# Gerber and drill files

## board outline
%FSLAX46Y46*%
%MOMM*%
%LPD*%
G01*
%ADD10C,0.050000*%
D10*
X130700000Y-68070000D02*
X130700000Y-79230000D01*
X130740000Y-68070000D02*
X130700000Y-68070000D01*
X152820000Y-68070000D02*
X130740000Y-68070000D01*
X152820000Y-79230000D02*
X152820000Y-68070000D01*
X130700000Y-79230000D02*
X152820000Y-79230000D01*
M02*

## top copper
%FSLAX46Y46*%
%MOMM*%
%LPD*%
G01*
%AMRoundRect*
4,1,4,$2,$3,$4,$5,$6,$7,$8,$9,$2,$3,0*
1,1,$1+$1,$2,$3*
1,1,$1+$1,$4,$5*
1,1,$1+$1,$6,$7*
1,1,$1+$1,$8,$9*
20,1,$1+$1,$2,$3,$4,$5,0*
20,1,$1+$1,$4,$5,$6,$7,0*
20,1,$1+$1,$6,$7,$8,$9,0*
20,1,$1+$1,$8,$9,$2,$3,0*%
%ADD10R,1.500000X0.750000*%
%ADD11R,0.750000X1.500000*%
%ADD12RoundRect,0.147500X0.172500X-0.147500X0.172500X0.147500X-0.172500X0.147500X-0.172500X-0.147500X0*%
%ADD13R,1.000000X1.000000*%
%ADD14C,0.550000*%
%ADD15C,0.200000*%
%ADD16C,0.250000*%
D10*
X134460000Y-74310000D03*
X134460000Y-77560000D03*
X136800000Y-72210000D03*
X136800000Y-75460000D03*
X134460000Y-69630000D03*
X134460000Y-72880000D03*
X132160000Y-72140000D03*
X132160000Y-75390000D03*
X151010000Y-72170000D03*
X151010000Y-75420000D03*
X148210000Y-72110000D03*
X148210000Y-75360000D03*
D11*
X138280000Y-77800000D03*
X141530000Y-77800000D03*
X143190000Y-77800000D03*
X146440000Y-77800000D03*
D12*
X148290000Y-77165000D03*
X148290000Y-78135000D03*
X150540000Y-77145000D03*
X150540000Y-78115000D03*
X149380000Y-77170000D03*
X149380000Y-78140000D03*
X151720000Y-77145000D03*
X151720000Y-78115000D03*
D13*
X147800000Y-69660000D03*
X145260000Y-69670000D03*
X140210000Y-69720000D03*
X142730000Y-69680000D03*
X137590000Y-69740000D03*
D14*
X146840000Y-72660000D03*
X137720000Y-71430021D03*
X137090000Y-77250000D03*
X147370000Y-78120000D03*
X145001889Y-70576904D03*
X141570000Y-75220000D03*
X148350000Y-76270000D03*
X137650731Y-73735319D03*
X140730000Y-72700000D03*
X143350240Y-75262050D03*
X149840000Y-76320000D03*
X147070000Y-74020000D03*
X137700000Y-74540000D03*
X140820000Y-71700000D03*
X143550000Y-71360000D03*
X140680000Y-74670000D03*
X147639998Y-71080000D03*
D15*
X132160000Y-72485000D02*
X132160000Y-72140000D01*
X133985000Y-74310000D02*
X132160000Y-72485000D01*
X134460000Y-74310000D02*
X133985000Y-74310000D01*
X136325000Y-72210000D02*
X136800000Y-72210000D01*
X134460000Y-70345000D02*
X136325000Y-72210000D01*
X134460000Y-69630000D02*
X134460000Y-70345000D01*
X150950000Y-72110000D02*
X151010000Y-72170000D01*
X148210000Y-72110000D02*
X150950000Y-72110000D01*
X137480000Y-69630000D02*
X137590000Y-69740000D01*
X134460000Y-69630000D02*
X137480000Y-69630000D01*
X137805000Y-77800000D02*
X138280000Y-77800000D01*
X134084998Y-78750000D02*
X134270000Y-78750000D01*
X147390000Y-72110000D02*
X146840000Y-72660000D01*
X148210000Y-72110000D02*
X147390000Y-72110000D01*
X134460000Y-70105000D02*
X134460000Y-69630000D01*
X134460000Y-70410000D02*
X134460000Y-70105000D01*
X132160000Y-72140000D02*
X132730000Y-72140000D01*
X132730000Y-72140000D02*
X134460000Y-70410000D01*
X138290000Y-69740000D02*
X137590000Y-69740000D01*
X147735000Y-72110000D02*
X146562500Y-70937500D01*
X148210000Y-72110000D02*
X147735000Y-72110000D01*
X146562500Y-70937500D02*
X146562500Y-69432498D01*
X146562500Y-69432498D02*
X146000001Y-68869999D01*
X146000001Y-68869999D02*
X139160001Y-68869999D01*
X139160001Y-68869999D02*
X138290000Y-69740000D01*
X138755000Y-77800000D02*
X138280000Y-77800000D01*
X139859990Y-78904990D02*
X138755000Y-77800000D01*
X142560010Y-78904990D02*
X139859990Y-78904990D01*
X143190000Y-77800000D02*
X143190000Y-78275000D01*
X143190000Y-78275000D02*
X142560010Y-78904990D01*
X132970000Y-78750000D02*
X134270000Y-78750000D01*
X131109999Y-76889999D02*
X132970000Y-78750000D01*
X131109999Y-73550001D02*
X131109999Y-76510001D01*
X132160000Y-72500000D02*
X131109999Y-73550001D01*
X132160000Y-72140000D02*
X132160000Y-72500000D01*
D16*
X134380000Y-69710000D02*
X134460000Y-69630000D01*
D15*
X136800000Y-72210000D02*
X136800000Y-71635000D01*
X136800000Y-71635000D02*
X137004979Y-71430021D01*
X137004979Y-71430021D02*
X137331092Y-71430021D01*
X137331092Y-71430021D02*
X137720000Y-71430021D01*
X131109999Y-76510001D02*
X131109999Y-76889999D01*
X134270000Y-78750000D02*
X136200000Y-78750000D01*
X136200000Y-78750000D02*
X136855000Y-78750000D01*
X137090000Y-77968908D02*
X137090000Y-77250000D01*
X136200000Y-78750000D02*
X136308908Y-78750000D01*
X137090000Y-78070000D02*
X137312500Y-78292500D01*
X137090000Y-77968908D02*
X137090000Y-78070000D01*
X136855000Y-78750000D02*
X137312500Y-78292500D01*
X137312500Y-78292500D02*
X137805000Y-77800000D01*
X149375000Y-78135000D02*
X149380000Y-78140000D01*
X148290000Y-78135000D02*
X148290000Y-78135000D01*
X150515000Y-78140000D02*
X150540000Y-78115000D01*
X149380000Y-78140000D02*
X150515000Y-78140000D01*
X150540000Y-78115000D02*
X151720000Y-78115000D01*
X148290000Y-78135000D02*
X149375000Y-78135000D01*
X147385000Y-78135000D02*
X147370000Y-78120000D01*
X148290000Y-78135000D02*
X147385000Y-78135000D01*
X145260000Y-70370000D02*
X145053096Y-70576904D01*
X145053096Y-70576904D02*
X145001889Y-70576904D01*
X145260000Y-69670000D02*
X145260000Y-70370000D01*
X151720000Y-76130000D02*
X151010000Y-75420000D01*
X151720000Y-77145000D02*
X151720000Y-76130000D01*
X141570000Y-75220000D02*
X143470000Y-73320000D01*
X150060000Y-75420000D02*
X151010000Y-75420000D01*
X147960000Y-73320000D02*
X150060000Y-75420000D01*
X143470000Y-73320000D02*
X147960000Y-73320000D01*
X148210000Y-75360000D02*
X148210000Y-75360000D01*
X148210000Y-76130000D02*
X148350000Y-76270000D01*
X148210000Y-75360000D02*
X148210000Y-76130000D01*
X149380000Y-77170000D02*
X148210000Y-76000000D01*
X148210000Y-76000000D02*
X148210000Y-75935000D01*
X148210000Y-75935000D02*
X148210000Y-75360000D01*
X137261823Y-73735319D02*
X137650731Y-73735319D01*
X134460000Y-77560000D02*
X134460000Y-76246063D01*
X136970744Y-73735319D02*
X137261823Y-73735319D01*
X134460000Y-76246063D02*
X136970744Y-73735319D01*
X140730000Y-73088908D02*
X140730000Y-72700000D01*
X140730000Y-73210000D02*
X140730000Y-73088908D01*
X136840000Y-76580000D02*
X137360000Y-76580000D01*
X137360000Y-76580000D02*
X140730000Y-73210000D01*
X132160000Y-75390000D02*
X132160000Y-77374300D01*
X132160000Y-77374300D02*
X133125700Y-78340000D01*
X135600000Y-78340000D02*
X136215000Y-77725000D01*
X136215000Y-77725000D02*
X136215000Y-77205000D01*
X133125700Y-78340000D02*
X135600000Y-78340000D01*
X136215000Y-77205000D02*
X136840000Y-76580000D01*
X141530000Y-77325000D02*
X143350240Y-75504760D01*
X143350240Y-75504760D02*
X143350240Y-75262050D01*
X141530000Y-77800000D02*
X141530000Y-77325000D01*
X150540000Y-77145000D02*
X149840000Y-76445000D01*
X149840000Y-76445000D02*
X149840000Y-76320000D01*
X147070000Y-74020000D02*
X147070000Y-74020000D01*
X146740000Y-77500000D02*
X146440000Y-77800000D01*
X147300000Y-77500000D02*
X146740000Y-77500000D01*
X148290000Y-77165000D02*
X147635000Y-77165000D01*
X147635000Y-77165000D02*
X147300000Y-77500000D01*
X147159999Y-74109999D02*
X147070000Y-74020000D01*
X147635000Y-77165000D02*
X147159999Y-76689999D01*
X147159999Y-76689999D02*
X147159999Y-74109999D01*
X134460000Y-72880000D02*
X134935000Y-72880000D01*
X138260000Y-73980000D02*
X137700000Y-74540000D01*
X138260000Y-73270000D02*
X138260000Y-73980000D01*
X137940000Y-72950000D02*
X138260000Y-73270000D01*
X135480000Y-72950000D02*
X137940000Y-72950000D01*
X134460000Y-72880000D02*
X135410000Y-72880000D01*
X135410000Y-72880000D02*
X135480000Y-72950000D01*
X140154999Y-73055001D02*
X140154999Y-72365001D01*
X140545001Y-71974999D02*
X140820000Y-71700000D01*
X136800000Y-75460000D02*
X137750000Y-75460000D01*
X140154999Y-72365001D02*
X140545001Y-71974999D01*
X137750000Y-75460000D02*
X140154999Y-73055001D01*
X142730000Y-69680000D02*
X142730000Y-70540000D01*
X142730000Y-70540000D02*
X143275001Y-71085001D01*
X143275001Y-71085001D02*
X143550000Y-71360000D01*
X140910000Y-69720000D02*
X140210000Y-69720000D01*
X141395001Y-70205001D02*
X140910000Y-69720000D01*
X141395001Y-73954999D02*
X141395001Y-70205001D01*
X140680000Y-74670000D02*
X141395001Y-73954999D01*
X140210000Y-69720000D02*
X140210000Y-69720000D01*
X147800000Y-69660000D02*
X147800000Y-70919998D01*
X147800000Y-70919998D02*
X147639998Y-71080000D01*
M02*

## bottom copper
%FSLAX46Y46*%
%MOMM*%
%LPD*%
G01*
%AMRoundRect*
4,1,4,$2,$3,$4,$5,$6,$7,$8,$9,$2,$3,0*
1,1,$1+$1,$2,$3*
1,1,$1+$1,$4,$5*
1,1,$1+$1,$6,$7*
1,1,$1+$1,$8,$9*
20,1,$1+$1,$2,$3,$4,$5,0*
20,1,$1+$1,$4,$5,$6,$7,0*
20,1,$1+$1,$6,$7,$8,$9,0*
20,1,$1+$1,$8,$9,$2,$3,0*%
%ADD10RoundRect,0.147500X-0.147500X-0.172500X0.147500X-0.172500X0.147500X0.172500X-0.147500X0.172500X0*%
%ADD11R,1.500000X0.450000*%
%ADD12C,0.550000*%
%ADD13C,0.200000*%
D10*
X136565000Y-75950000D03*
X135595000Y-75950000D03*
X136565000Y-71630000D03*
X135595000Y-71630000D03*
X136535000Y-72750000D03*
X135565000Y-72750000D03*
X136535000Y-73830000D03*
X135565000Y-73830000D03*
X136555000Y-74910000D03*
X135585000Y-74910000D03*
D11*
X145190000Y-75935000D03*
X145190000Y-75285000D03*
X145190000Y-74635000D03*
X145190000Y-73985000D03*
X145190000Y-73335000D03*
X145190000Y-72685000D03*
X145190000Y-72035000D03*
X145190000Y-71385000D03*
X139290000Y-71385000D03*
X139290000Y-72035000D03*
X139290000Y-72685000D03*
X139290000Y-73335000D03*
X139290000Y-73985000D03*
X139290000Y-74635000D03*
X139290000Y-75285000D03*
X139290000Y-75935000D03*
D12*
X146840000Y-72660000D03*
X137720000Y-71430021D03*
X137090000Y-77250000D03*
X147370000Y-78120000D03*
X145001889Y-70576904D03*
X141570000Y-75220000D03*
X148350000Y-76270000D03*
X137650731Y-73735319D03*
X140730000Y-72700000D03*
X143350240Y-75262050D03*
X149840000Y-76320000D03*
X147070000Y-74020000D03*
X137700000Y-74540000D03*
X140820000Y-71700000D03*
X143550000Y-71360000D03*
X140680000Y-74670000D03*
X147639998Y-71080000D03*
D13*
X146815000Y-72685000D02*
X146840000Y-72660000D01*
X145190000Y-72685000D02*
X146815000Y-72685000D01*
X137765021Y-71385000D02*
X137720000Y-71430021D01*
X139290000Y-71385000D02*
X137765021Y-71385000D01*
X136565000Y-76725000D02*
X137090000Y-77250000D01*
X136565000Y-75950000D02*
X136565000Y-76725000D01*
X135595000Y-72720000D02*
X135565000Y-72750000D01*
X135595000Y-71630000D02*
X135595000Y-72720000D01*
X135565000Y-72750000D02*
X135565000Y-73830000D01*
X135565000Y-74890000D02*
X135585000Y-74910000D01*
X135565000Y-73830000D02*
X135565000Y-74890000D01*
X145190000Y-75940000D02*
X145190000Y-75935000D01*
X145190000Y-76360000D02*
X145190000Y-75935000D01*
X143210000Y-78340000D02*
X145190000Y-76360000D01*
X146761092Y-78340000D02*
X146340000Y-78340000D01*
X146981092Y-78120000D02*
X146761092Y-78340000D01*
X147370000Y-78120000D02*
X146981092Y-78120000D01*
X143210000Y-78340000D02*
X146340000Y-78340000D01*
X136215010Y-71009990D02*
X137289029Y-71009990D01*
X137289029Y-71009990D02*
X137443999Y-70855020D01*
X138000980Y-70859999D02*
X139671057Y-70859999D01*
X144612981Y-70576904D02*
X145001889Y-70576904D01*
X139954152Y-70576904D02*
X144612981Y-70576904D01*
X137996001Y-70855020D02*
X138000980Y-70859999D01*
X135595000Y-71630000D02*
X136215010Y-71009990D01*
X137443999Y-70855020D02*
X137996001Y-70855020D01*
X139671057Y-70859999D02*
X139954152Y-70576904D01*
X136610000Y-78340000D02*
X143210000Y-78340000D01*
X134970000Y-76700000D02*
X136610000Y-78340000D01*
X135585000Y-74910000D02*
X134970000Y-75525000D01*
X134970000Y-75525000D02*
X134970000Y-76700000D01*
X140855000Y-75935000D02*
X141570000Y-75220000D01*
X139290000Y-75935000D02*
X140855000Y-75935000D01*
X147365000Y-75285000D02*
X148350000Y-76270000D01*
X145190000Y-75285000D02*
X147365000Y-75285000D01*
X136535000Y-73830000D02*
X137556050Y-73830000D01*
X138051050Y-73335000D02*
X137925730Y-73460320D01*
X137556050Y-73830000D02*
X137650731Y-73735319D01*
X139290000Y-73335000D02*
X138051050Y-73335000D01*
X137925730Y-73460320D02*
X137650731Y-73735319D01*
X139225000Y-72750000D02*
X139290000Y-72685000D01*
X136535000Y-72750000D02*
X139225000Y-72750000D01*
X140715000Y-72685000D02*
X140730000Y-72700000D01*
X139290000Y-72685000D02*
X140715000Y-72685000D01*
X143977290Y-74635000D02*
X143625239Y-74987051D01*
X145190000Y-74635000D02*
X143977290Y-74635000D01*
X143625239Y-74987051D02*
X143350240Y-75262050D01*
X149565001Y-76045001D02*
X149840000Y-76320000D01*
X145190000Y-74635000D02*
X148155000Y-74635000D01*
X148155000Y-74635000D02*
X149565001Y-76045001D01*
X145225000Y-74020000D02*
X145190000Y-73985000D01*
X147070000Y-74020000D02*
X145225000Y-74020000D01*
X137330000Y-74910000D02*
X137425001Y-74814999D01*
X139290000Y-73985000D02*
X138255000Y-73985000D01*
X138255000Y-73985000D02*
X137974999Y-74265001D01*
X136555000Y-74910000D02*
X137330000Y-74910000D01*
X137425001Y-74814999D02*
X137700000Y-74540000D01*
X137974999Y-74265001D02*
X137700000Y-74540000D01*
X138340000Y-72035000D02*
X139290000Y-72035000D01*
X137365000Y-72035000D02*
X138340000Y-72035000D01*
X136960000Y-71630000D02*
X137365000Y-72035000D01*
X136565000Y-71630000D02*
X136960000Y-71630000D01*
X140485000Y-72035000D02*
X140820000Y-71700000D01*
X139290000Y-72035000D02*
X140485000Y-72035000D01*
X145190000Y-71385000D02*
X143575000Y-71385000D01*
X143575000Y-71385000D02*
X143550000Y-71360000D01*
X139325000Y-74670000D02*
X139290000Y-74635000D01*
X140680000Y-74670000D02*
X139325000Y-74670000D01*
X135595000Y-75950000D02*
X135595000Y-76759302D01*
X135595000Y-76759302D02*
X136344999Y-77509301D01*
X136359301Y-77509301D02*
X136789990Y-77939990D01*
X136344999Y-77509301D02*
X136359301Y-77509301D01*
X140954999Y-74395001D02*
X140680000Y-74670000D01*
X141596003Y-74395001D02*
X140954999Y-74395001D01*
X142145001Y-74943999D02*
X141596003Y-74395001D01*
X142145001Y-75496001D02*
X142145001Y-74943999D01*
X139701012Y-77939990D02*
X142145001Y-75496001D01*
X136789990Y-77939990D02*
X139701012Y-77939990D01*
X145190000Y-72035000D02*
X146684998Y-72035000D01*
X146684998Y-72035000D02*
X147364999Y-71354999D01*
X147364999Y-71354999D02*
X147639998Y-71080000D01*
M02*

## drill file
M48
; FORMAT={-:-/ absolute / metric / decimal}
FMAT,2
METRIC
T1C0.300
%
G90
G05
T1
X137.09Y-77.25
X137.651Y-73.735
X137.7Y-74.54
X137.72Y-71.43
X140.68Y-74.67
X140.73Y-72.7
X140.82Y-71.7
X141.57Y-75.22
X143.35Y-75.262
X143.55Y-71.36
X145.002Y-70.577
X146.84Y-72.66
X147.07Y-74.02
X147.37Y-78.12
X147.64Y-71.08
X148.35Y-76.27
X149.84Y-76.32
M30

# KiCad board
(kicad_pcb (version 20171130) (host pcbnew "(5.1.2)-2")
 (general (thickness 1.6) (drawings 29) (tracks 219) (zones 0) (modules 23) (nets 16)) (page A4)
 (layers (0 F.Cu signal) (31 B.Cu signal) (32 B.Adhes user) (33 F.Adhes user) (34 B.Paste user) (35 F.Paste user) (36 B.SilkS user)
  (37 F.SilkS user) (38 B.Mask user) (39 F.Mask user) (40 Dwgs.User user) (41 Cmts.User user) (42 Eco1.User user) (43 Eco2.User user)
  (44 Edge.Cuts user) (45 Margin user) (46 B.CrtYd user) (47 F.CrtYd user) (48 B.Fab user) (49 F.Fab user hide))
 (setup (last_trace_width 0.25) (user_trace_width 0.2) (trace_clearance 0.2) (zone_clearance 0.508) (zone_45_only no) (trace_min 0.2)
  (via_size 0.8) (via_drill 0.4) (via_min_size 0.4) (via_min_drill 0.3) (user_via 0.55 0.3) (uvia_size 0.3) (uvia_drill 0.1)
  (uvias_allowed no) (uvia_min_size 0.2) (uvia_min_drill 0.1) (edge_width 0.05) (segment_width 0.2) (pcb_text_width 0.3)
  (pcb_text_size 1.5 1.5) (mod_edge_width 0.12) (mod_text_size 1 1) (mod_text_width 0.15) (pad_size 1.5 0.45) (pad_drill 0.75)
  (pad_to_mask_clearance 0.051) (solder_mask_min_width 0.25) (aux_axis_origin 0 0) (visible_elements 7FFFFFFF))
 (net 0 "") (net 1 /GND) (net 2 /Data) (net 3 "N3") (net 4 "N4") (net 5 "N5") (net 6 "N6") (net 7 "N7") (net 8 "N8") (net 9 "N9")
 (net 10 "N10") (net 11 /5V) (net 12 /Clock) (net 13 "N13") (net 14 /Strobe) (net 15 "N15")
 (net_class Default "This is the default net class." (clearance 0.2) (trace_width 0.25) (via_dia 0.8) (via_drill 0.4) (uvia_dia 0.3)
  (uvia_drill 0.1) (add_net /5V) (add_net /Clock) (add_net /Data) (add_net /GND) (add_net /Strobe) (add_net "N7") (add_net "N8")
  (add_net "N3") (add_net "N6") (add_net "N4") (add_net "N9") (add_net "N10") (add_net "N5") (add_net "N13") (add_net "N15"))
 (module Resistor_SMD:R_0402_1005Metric (layer B.Cu) (at 136.08 75.95)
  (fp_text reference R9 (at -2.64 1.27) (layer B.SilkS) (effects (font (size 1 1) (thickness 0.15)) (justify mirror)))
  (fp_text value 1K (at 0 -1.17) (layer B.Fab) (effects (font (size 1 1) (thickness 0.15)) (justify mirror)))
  (pad 2 smd roundrect (at 0.485 0) (size 0.59 0.64) (layers B.Cu B.Paste B.Mask) (roundrect_rratio 0.25) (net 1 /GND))
  (pad 1 smd roundrect (at -0.485 0) (size 0.59 0.64) (layers B.Cu B.Paste B.Mask) (roundrect_rratio 0.25) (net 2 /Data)))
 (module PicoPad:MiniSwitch (layer F.Cu) (at 131.92 78.83 90)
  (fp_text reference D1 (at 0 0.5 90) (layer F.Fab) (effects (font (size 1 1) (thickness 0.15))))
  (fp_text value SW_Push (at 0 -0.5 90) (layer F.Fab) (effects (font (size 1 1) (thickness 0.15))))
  (pad 1 smd rect (at 4.52 2.54 90) (size 0.75 1.5) (layers F.Cu F.Paste F.Mask) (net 1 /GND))
  (pad 2 smd rect (at 1.27 2.54 90) (size 0.75 1.5) (layers F.Cu F.Paste F.Mask) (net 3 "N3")))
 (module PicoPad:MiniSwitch (layer F.Cu) (at 134.26 76.73 90)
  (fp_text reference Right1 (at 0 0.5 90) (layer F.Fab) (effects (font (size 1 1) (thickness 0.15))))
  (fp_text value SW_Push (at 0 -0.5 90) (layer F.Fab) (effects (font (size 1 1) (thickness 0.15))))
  (pad 1 smd rect (at 4.52 2.54 90) (size 0.75 1.5) (layers F.Cu F.Paste F.Mask) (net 1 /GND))
  (pad 2 smd rect (at 1.27 2.54 90) (size 0.75 1.5) (layers F.Cu F.Paste F.Mask) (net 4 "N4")))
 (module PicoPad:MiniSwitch (layer F.Cu) (at 131.92 74.15 90)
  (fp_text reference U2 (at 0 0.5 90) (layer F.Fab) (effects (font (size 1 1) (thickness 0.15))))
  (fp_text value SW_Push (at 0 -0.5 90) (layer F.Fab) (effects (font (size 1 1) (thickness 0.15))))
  (pad 1 smd rect (at 4.52 2.54 90) (size 0.75 1.5) (layers F.Cu F.Paste F.Mask) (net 1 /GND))
  (pad 2 smd rect (at 1.27 2.54 90) (size 0.75 1.5) (layers F.Cu F.Paste F.Mask) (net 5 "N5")))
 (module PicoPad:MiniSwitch (layer F.Cu) (at 129.62 76.66 90)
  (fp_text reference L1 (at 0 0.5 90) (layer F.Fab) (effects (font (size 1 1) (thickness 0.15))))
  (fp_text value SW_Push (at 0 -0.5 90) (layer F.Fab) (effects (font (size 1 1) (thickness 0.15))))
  (pad 1 smd rect (at 4.52 2.54 90) (size 0.75 1.5) (layers F.Cu F.Paste F.Mask) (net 1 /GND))
  (pad 2 smd rect (at 1.27 2.54 90) (size 0.75 1.5) (layers F.Cu F.Paste F.Mask) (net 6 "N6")))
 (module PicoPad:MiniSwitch (layer F.Cu) (at 148.47 76.69 90)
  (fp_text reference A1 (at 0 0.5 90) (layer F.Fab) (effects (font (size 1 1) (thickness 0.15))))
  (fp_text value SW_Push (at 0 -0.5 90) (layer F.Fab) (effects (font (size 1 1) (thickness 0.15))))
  (pad 1 smd rect (at 4.52 2.54 90) (size 0.75 1.5) (layers F.Cu F.Paste F.Mask) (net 1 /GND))
  (pad 2 smd rect (at 1.27 2.54 90) (size 0.75 1.5) (layers F.Cu F.Paste F.Mask) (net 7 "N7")))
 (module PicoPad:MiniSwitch (layer F.Cu) (at 145.67 76.63 90)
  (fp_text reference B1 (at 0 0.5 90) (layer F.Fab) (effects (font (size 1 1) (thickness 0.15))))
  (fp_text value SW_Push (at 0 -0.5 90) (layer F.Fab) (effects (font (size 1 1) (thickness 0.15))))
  (pad 1 smd rect (at 4.52 2.54 90) (size 0.75 1.5) (layers F.Cu F.Paste F.Mask) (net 1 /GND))
  (pad 2 smd rect (at 1.27 2.54 90) (size 0.75 1.5) (layers F.Cu F.Paste F.Mask) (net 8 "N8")))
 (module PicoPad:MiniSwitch (layer F.Cu) (at 142.8 80.34 180)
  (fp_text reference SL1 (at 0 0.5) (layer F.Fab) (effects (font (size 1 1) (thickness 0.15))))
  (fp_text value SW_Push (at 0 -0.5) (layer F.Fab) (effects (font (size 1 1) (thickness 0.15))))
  (pad 1 smd rect (at 4.52 2.54 180) (size 0.75 1.5) (layers F.Cu F.Paste F.Mask) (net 1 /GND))
  (pad 2 smd rect (at 1.27 2.54 180) (size 0.75 1.5) (layers F.Cu F.Paste F.Mask) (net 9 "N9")))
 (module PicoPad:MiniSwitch (layer F.Cu) (at 147.71 80.34 180)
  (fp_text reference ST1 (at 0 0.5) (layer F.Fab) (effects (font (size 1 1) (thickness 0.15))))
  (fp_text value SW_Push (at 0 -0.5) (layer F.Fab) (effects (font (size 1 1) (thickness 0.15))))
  (pad 1 smd rect (at 4.52 2.54 180) (size 0.75 1.5) (layers F.Cu F.Paste F.Mask) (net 1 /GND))
  (pad 2 smd rect (at 1.27 2.54 180) (size 0.75 1.5) (layers F.Cu F.Paste F.Mask) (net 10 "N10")))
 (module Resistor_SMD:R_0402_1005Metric (layer B.Cu) (at 136.08 71.63)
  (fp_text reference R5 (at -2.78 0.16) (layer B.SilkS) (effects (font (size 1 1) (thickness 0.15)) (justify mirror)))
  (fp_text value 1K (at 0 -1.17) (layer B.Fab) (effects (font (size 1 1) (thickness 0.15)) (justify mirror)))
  (pad 2 smd roundrect (at 0.485 0) (size 0.59 0.64) (layers B.Cu B.Paste B.Mask) (roundrect_rratio 0.25) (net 4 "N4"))
  (pad 1 smd roundrect (at -0.485 0) (size 0.59 0.64) (layers B.Cu B.Paste B.Mask) (roundrect_rratio 0.25) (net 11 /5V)))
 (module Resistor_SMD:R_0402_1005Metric (layer B.Cu) (at 136.05 72.75)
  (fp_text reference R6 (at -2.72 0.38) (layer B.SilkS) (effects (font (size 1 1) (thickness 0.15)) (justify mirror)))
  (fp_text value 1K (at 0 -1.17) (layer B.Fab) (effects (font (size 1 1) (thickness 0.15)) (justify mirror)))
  (pad 2 smd roundrect (at 0.485 0) (size 0.59 0.64) (layers B.Cu B.Paste B.Mask) (roundrect_rratio 0.25) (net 6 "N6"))
  (pad 1 smd roundrect (at -0.485 0) (size 0.59 0.64) (layers B.Cu B.Paste B.Mask) (roundrect_rratio 0.25) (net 11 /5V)))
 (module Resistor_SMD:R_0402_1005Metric (layer B.Cu) (at 136.05 73.83)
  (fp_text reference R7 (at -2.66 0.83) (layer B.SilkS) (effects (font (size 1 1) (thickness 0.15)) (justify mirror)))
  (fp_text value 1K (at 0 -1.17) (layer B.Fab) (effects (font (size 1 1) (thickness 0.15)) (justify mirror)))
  (pad 2 smd roundrect (at 0.485 0) (size 0.59 0.64) (layers B.Cu B.Paste B.Mask) (roundrect_rratio 0.25) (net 3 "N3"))
  (pad 1 smd roundrect (at -0.485 0) (size 0.59 0.64) (layers B.Cu B.Paste B.Mask) (roundrect_rratio 0.25) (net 11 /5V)))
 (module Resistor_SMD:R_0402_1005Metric (layer B.Cu) (at 136.07 74.91)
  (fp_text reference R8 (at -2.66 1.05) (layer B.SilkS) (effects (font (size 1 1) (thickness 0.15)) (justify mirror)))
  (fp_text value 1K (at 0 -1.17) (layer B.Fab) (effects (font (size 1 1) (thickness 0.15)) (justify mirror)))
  (pad 2 smd roundrect (at 0.485 0) (size 0.59 0.64) (layers B.Cu B.Paste B.Mask) (roundrect_rratio 0.25) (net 5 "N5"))
  (pad 1 smd roundrect (at -0.485 0) (size 0.59 0.64) (layers B.Cu B.Paste B.Mask) (roundrect_rratio 0.25) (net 11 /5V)))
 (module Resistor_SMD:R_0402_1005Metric (layer F.Cu) (at 148.29 77.65 90)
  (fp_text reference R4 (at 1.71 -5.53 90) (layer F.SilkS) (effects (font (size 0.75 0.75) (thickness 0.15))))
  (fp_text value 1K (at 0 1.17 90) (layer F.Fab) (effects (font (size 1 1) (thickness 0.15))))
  (pad 2 smd roundrect (at 0.485 0 90) (size 0.59 0.64) (layers F.Cu F.Paste F.Mask) (roundrect_rratio 0.25) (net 10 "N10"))
  (pad 1 smd roundrect (at -0.485 0 90) (size 0.59 0.64) (layers F.Cu F.Paste F.Mask) (roundrect_rratio 0.25) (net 11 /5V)))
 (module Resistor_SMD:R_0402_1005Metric (layer F.Cu) (at 150.54 77.63 90)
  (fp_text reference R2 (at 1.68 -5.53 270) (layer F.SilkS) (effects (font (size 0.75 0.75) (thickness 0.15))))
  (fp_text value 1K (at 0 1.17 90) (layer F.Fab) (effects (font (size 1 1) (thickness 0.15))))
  (pad 2 smd roundrect (at 0.485 0 90) (size 0.59 0.64) (layers F.Cu F.Paste F.Mask) (roundrect_rratio 0.25) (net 9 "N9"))
  (pad 1 smd roundrect (at -0.485 0 90) (size 0.59 0.64) (layers F.Cu F.Paste F.Mask) (roundrect_rratio 0.25) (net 11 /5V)))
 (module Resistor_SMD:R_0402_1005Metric (layer F.Cu) (at 149.38 77.655 90)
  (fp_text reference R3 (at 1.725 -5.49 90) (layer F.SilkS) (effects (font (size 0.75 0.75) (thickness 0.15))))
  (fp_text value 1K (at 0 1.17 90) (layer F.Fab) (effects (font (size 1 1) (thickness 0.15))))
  (pad 2 smd roundrect (at 0.485 0 90) (size 0.59 0.64) (layers F.Cu F.Paste F.Mask) (roundrect_rratio 0.25) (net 8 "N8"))
  (pad 1 smd roundrect (at -0.485 0 90) (size 0.59 0.64) (layers F.Cu F.Paste F.Mask) (roundrect_rratio 0.25) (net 11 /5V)))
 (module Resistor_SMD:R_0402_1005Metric (layer F.Cu) (at 151.72 77.63 90)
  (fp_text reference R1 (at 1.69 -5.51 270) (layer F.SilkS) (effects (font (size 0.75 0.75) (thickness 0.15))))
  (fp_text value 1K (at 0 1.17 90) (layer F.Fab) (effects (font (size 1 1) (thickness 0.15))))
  (pad 2 smd roundrect (at 0.485 0 90) (size 0.59 0.64) (layers F.Cu F.Paste F.Mask) (roundrect_rratio 0.25) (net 7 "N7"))
  (pad 1 smd roundrect (at -0.485 0 90) (size 0.59 0.64) (layers F.Cu F.Paste F.Mask) (roundrect_rratio 0.25) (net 11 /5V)))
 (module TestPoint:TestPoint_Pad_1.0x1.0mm (layer F.Cu) (at 147.8 69.66)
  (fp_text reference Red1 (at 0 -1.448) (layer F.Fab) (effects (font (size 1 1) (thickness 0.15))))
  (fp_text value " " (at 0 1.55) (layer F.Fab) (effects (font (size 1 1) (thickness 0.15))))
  (pad 1 smd rect (at 0 0) (size 1 1) (layers F.Cu F.Mask) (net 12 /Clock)))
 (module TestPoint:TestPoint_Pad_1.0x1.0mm (layer F.Cu) (at 145.26 69.67)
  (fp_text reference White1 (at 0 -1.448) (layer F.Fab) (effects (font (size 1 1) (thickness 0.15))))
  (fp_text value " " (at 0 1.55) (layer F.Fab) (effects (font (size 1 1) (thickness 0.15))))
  (pad 1 smd rect (at 0 0) (size 1 1) (layers F.Cu F.Mask) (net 11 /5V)))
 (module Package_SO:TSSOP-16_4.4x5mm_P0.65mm (layer B.Cu) (at 142.24 73.66)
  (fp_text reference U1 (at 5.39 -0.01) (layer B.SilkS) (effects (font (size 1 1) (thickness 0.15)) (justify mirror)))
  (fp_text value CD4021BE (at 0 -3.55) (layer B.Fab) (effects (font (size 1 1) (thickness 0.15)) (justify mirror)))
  (pad 16 smd rect (at 2.95 2.275) (size 1.5 0.45) (layers B.Cu B.Paste B.Mask) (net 11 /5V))
  (pad 15 smd rect (at 2.95 1.625) (size 1.5 0.45) (layers B.Cu B.Paste B.Mask) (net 8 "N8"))
  (pad 14 smd rect (at 2.95 0.975) (size 1.5 0.45) (layers B.Cu B.Paste B.Mask) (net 9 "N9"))
  (pad 13 smd rect (at 2.95 0.325) (size 1.5 0.45) (layers B.Cu B.Paste B.Mask) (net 10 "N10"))
  (pad 12 smd rect (at 2.95 -0.325) (size 1.5 0.45) (layers B.Cu B.Paste B.Mask) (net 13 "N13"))
  (pad 11 smd rect (at 2.95 -0.975) (size 1.5 0.45) (layers B.Cu B.Paste B.Mask) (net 1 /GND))
  (pad 10 smd rect (at 2.95 -1.625) (size 1.5 0.45) (layers B.Cu B.Paste B.Mask) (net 12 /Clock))
  (pad 9 smd rect (at 2.95 -2.275) (size 1.5 0.45) (layers B.Cu B.Paste B.Mask) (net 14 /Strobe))
  (pad 8 smd rect (at -2.95 -2.275) (size 1.5 0.45) (layers B.Cu B.Paste B.Mask) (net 1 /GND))
  (pad 7 smd rect (at -2.95 -1.625) (size 1.5 0.45) (layers B.Cu B.Paste B.Mask) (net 4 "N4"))
  (pad 6 smd rect (at -2.95 -0.975) (size 1.5 0.45) (layers B.Cu B.Paste B.Mask) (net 6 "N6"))
  (pad 5 smd rect (at -2.95 -0.325) (size 1.5 0.45) (layers B.Cu B.Paste B.Mask) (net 3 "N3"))
  (pad 4 smd rect (at -2.95 0.325) (size 1.5 0.45) (layers B.Cu B.Paste B.Mask) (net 5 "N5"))
  (pad 3 smd rect (at -2.95 0.975) (size 1.5 0.45) (layers B.Cu B.Paste B.Mask) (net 2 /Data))
  (pad 2 smd rect (at -2.95 1.625) (size 1.5 0.45) (layers B.Cu B.Paste B.Mask) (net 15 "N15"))
  (pad 1 smd rect (at -2.95 2.275) (size 1.5 0.45) (layers B.Cu B.Paste B.Mask) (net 7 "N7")))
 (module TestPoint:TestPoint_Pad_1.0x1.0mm (layer F.Cu) (at 140.21 69.72)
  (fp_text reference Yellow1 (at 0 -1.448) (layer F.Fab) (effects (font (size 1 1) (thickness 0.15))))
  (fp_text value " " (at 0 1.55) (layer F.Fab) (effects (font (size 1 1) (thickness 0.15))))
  (pad 1 smd rect (at 0 0) (size 1 1) (layers F.Cu F.Mask) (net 2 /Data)))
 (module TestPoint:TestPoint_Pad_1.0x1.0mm (layer F.Cu) (at 142.73 69.68)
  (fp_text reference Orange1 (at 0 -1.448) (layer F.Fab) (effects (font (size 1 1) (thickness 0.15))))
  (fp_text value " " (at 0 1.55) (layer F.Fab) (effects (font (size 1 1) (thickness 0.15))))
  (pad 1 smd rect (at 0 0) (size 1 1) (layers F.Cu F.Mask) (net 14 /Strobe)))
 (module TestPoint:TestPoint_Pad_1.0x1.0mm (layer F.Cu) (at 137.59 69.74)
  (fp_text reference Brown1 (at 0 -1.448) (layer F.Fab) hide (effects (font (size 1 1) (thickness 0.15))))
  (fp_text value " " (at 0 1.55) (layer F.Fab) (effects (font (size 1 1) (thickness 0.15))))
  (pad 1 smd rect (at 0 0) (size 1 1) (layers F.Cu F.Mask) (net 1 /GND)))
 (gr_line (start 130.7 68.07) (end 130.7 79.23) (layer Edge.Cuts) (width 0.05))
 (gr_line (start 130.74 68.07) (end 130.7 68.07) (layer Edge.Cuts) (width 0.05))
 (gr_line (start 152.82 68.07) (end 130.74 68.07) (layer Edge.Cuts) (width 0.05))
 (gr_line (start 152.82 79.23) (end 152.82 68.07) (layer Edge.Cuts) (width 0.05))
 (gr_line (start 130.7 79.23) (end 152.82 79.23) (layer Edge.Cuts) (width 0.05))
 (via (at 146.84 72.66) (size 0.55) (drill 0.3) (layers F.Cu B.Cu) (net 1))
 (segment (start 132.16 72.485) (end 132.16 72.14) (width 0.2) (layer F.Cu) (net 1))
 (segment (start 133.985 74.31) (end 132.16 72.485) (width 0.2) (layer F.Cu) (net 1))
 (segment (start 134.46 74.31) (end 133.985 74.31) (width 0.2) (layer F.Cu) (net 1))
 (segment (start 136.325 72.21) (end 136.8 72.21) (width 0.2) (layer F.Cu) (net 1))
 (segment (start 134.46 70.345) (end 136.325 72.21) (width 0.2) (layer F.Cu) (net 1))
 (segment (start 134.46 69.63) (end 134.46 70.345) (width 0.2) (layer F.Cu) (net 1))
 (segment (start 150.95 72.11) (end 151.01 72.17) (width 0.2) (layer F.Cu) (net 1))
 (segment (start 148.21 72.11) (end 150.95 72.11) (width 0.2) (layer F.Cu) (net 1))
 (segment (start 137.48 69.63) (end 137.59 69.74) (width 0.2) (layer F.Cu) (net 1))
 (segment (start 134.46 69.63) (end 137.48 69.63) (width 0.2) (layer F.Cu) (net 1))
 (segment (start 137.805 77.8) (end 138.28 77.8) (width 0.2) (layer F.Cu) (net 1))
 (segment (start 134.084998 78.75) (end 134.27 78.75) (width 0.2) (layer F.Cu) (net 1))
 (segment (start 146.815 72.685) (end 146.84 72.66) (width 0.2) (layer B.Cu) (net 1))
 (segment (start 145.19 72.685) (end 146.815 72.685) (width 0.2) (layer B.Cu) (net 1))
 (segment (start 147.39 72.11) (end 146.84 72.66) (width 0.2) (layer F.Cu) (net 1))
 (segment (start 148.21 72.11) (end 147.39 72.11) (width 0.2) (layer F.Cu) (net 1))
 (segment (start 134.46 70.105) (end 134.46 69.63) (width 0.2) (layer F.Cu) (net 1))
 (segment (start 134.46 70.41) (end 134.46 70.105) (width 0.2) (layer F.Cu) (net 1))
 (segment (start 132.16 72.14) (end 132.73 72.14) (width 0.2) (layer F.Cu) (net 1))
 (segment (start 132.73 72.14) (end 134.46 70.41) (width 0.2) (layer F.Cu) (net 1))
 (segment (start 138.29 69.74) (end 137.59 69.74) (width 0.2) (layer F.Cu) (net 1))
 (segment (start 147.735 72.11) (end 146.5625 70.9375) (width 0.2) (layer F.Cu) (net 1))
 (segment (start 148.21 72.11) (end 147.735 72.11) (width 0.2) (layer F.Cu) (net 1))
 (segment (start 146.5625 70.9375) (end 146.5625 69.432498) (width 0.2) (layer F.Cu) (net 1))
 (segment (start 146.5625 69.432498) (end 146.000001 68.869999) (width 0.2) (layer F.Cu) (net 1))
 (segment (start 146.000001 68.869999) (end 139.160001 68.869999) (width 0.2) (layer F.Cu) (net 1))
 (segment (start 139.160001 68.869999) (end 138.29 69.74) (width 0.2) (layer F.Cu) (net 1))
 (segment (start 138.755 77.8) (end 138.28 77.8) (width 0.2) (layer F.Cu) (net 1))
 (segment (start 139.85999 78.90499) (end 138.755 77.8) (width 0.2) (layer F.Cu) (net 1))
 (segment (start 142.56001 78.90499) (end 139.85999 78.90499) (width 0.2) (layer F.Cu) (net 1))
 (segment (start 143.19 77.8) (end 143.19 78.275) (width 0.2) (layer F.Cu) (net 1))
 (segment (start 143.19 78.275) (end 142.56001 78.90499) (width 0.2) (layer F.Cu) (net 1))
 (segment (start 132.97 78.75) (end 134.27 78.75) (width 0.2) (layer F.Cu) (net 1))
 (segment (start 131.109999 76.889999) (end 132.97 78.75) (width 0.2) (layer F.Cu) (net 1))
 (segment (start 131.109999 73.550001) (end 131.109999 76.510001) (width 0.2) (layer F.Cu) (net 1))
 (segment (start 132.16 72.5) (end 131.109999 73.550001) (width 0.2) (layer F.Cu) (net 1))
 (segment (start 132.16 72.14) (end 132.16 72.5) (width 0.2) (layer F.Cu) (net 1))
 (segment (start 134.38 69.71) (end 134.46 69.63) (width 0.25) (layer F.Cu) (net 1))
 (segment (start 137.765021 71.385) (end 137.72 71.430021) (width 0.2) (layer B.Cu) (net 1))
 (segment (start 136.8 72.21) (end 136.8 71.635) (width 0.2) (layer F.Cu) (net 1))
 (segment (start 136.8 71.635) (end 137.004979 71.430021) (width 0.2) (layer F.Cu) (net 1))
 (segment (start 137.004979 71.430021) (end 137.331092 71.430021) (width 0.2) (layer F.Cu) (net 1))
 (via (at 137.72 71.430021) (size 0.55) (drill 0.3) (layers F.Cu B.Cu) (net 1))
 (segment (start 137.331092 71.430021) (end 137.72 71.430021) (width 0.2) (layer F.Cu) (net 1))
 (segment (start 139.29 71.385) (end 137.765021 71.385) (width 0.2) (layer B.Cu) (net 1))
 (segment (start 131.109999 76.510001) (end 131.109999 76.889999) (width 0.2) (layer F.Cu) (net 1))
 (via (at 137.09 77.25) (size 0.55) (drill 0.3) (layers F.Cu B.Cu) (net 1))
 (segment (start 134.27 78.75) (end 136.2 78.75) (width 0.2) (layer F.Cu) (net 1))
 (segment (start 136.2 78.75) (end 136.855 78.75) (width 0.2) (layer F.Cu) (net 1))
 (segment (start 136.565 76.725) (end 137.09 77.25) (width 0.2) (layer B.Cu) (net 1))
 (segment (start 136.565 75.95) (end 136.565 76.725) (width 0.2) (layer B.Cu) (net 1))
 (segment (start 137.09 77.968908) (end 137.09 77.25) (width 0.2) (layer F.Cu) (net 1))
 (segment (start 136.2 78.75) (end 136.308908 78.75) (width 0.2) (layer F.Cu) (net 1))
 (segment (start 137.09 78.07) (end 137.3125 78.2925) (width 0.2) (layer F.Cu) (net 1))
 (segment (start 137.09 77.968908) (end 137.09 78.07) (width 0.2) (layer F.Cu) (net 1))
 (segment (start 136.855 78.75) (end 137.3125 78.2925) (width 0.2) (layer F.Cu) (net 1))
 (segment (start 137.3125 78.2925) (end 137.805 77.8) (width 0.2) (layer F.Cu) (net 1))
 (segment (start 149.375 78.135) (end 149.38 78.14) (width 0.2) (layer F.Cu) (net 11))
 (segment (start 148.29 78.135) (end 148.29 78.135) (width 0.2) (layer F.Cu) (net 11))
 (segment (start 150.515 78.14) (end 150.54 78.115) (width 0.2) (layer F.Cu) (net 11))
 (segment (start 149.38 78.14) (end 150.515 78.14) (width 0.2) (layer F.Cu) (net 11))
 (segment (start 150.54 78.115) (end 151.72 78.115) (width 0.2) (layer F.Cu) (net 11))
 (segment (start 135.595 72.72) (end 135.565 72.75) (width 0.2) (layer B.Cu) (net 11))
 (segment (start 135.595 71.63) (end 135.595 72.72) (width 0.2) (layer B.Cu) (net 11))
 (segment (start 135.565 72.75) (end 135.565 73.83) (width 0.2) (layer B.Cu) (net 11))
 (segment (start 135.565 74.89) (end 135.585 74.91) (width 0.2) (layer B.Cu) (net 11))
 (segment (start 135.565 73.83) (end 135.565 74.89) (width 0.2) (layer B.Cu) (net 11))
 (segment (start 148.29 78.135) (end 149.375 78.135) (width 0.2) (layer F.Cu) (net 11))
 (via (at 147.37 78.12) (size 0.55) (drill 0.3) (layers F.Cu B.Cu) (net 11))
 (segment (start 145.19 75.94) (end 145.19 75.935) (width 0.2) (layer B.Cu) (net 11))
 (segment (start 147.385 78.135) (end 147.37 78.12) (width 0.2) (layer F.Cu) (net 11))
 (segment (start 148.29 78.135) (end 147.385 78.135) (width 0.2) (layer F.Cu) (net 11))
 (segment (start 145.19 76.36) (end 145.19 75.935) (width 0.2) (layer B.Cu) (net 11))
 (segment (start 143.21 78.34) (end 145.19 76.36) (width 0.2) (layer B.Cu) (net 11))
 (segment (start 146.761092 78.34) (end 146.34 78.34) (width 0.2) (layer B.Cu) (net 11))
 (segment (start 146.981092 78.12) (end 146.761092 78.34) (width 0.2) (layer B.Cu) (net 11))
 (segment (start 147.37 78.12) (end 146.981092 78.12) (width 0.2) (layer B.Cu) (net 11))
 (segment (start 143.21 78.34) (end 146.34 78.34) (width 0.2) (layer B.Cu) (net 11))
 (segment (start 145.26 70.37) (end 145.053096 70.576904) (width 0.2) (layer F.Cu) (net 11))
 (via (at 145.001889 70.576904) (size 0.55) (drill 0.3) (layers F.Cu B.Cu) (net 11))
 (segment (start 145.053096 70.576904) (end 145.001889 70.576904) (width 0.2) (layer F.Cu) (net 11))
 (segment (start 145.26 69.67) (end 145.26 70.37) (width 0.2) (layer F.Cu) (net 11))
 (segment (start 136.21501 71.00999) (end 137.289029 71.00999) (width 0.2) (layer B.Cu) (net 11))
 (segment (start 137.289029 71.00999) (end 137.443999 70.85502) (width 0.2) (layer B.Cu) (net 11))
 (segment (start 138.00098 70.859999) (end 139.671057 70.859999) (width 0.2) (layer B.Cu) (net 11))
 (segment (start 144.612981 70.576904) (end 145.001889 70.576904) (width 0.2) (layer B.Cu) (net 11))
 (segment (start 139.954152 70.576904) (end 144.612981 70.576904) (width 0.2) (layer B.Cu) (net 11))
 (segment (start 137.996001 70.85502) (end 138.00098 70.859999) (width 0.2) (layer B.Cu) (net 11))
 (segment (start 135.595 71.63) (end 136.21501 71.00999) (width 0.2) (layer B.Cu) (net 11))
 (segment (start 137.443999 70.85502) (end 137.996001 70.85502) (width 0.2) (layer B.Cu) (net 11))
 (segment (start 139.671057 70.859999) (end 139.954152 70.576904) (width 0.2) (layer B.Cu) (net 11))
 (segment (start 136.61 78.34) (end 143.21 78.34) (width 0.2) (layer B.Cu) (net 11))
 (segment (start 134.97 76.7) (end 136.61 78.34) (width 0.2) (layer B.Cu) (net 11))
 (segment (start 135.585 74.91) (end 134.97 75.525) (width 0.2) (layer B.Cu) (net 11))
 (segment (start 134.97 75.525) (end 134.97 76.7) (width 0.2) (layer B.Cu) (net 11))
 (via (at 141.57 75.22) (size 0.55) (drill 0.3) (layers F.Cu B.Cu) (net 7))
 (segment (start 151.72 76.13) (end 151.01 75.42) (width 0.2) (layer F.Cu) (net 7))
 (segment (start 151.72 77.145) (end 151.72 76.13) (width 0.2) (layer F.Cu) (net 7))
 (segment (start 140.855 75.935) (end 141.57 75.22) (width 0.2) (layer B.Cu) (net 7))
 (segment (start 139.29 75.935) (end 140.855 75.935) (width 0.2) (layer B.Cu) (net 7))
 (segment (start 141.57 75.22) (end 143.47 73.32) (width 0.2) (layer F.Cu) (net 7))
 (segment (start 150.06 75.42) (end 151.01 75.42) (width 0.2) (layer F.Cu) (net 7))
 (segment (start 147.96 73.32) (end 150.06 75.42) (width 0.2) (layer F.Cu) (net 7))
 (segment (start 143.47 73.32) (end 147.96 73.32) (width 0.2) (layer F.Cu) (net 7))
 (segment (start 148.21 75.36) (end 148.21 75.36) (width 0.2) (layer F.Cu) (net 8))
 (via (at 148.35 76.27) (size 0.55) (drill 0.3) (layers F.Cu B.Cu) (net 8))
 (segment (start 147.365 75.285) (end 148.35 76.27) (width 0.2) (layer B.Cu) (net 8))
 (segment (start 145.19 75.285) (end 147.365 75.285) (width 0.2) (layer B.Cu) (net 8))
 (segment (start 148.21 76.13) (end 148.35 76.27) (width 0.2) (layer F.Cu) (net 8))
 (segment (start 148.21 75.36) (end 148.21 76.13) (width 0.2) (layer F.Cu) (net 8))
 (segment (start 149.38 77.17) (end 148.21 76) (width 0.2) (layer F.Cu) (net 8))
 (segment (start 148.21 76) (end 148.21 75.935) (width 0.2) (layer F.Cu) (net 8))
 (segment (start 148.21 75.935) (end 148.21 75.36) (width 0.2) (layer F.Cu) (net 8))
 (segment (start 136.535 73.83) (end 137.55605 73.83) (width 0.2) (layer B.Cu) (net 3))
 (segment (start 137.261823 73.735319) (end 137.650731 73.735319) (width 0.2) (layer F.Cu) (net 3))
 (segment (start 134.46 77.56) (end 134.46 76.246063) (width 0.2) (layer F.Cu) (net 3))
 (segment (start 136.970744 73.735319) (end 137.261823 73.735319) (width 0.2) (layer F.Cu) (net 3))
 (segment (start 138.05105 73.335) (end 137.92573 73.46032) (width 0.2) (layer B.Cu) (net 3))
 (segment (start 134.46 76.246063) (end 136.970744 73.735319) (width 0.2) (layer F.Cu) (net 3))
 (segment (start 137.55605 73.83) (end 137.650731 73.735319) (width 0.2) (layer B.Cu) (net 3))
 (segment (start 139.29 73.335) (end 138.05105 73.335) (width 0.2) (layer B.Cu) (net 3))
 (segment (start 137.92573 73.46032) (end 137.650731 73.735319) (width 0.2) (layer B.Cu) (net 3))
 (via (at 137.650731 73.735319) (size 0.55) (drill 0.3) (layers F.Cu B.Cu) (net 3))
 (via (at 140.73 72.7) (size 0.55) (drill 0.3) (layers F.Cu B.Cu) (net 6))
 (segment (start 139.225 72.75) (end 139.29 72.685) (width 0.2) (layer B.Cu) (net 6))
 (segment (start 136.535 72.75) (end 139.225 72.75) (width 0.2) (layer B.Cu) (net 6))
 (segment (start 140.715 72.685) (end 140.73 72.7) (width 0.2) (layer B.Cu) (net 6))
 (segment (start 139.29 72.685) (end 140.715 72.685) (width 0.2) (layer B.Cu) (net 6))
 (segment (start 140.73 73.088908) (end 140.73 72.7) (width 0.2) (layer F.Cu) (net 6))
 (segment (start 140.73 73.21) (end 140.73 73.088908) (width 0.2) (layer F.Cu) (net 6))
 (segment (start 136.84 76.58) (end 137.36 76.58) (width 0.2) (layer F.Cu) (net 6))
 (segment (start 137.36 76.58) (end 140.73 73.21) (width 0.2) (layer F.Cu) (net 6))
 (segment (start 132.16 75.39) (end 132.16 77.3743) (width 0.2) (layer F.Cu) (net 6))
 (segment (start 132.16 77.3743) (end 133.1257 78.34) (width 0.2) (layer F.Cu) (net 6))
 (segment (start 135.6 78.34) (end 136.215 77.725) (width 0.2) (layer F.Cu) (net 6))
 (segment (start 136.215 77.725) (end 136.215 77.205) (width 0.2) (layer F.Cu) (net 6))
 (segment (start 133.1257 78.34) (end 135.6 78.34) (width 0.2) (layer F.Cu) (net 6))
 (segment (start 136.215 77.205) (end 136.84 76.58) (width 0.2) (layer F.Cu) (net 6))
 (via (at 143.35024 75.26205) (size 0.55) (drill 0.3) (layers F.Cu B.Cu) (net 9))
 (segment (start 141.53 77.325) (end 143.35024 75.50476) (width 0.2) (layer F.Cu) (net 9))
 (segment (start 143.35024 75.50476) (end 143.35024 75.26205) (width 0.2) (layer F.Cu) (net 9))
 (segment (start 141.53 77.8) (end 141.53 77.325) (width 0.2) (layer F.Cu) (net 9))
 (segment (start 143.97729 74.635) (end 143.625239 74.987051) (width 0.2) (layer B.Cu) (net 9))
 (segment (start 145.19 74.635) (end 143.97729 74.635) (width 0.2) (layer B.Cu) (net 9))
 (segment (start 143.625239 74.987051) (end 143.35024 75.26205) (width 0.2) (layer B.Cu) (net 9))
 (via (at 149.84 76.32) (size 0.55) (drill 0.3) (layers F.Cu B.Cu) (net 9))
 (segment (start 150.54 77.145) (end 149.84 76.445) (width 0.2) (layer F.Cu) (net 9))
 (segment (start 149.565001 76.045001) (end 149.84 76.32) (width 0.2) (layer B.Cu) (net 9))
 (segment (start 145.19 74.635) (end 148.155 74.635) (width 0.2) (layer B.Cu) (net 9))
 (segment (start 148.155 74.635) (end 149.565001 76.045001) (width 0.2) (layer B.Cu) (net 9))
 (segment (start 149.84 76.445) (end 149.84 76.32) (width 0.2) (layer F.Cu) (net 9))
 (segment (start 147.07 74.02) (end 147.07 74.02) (width 0.2) (layer F.Cu) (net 10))
 (via (at 147.07 74.02) (size 0.55) (drill 0.3) (layers F.Cu B.Cu) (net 10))
 (segment (start 145.225 74.02) (end 145.19 73.985) (width 0.2) (layer B.Cu) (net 10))
 (segment (start 147.07 74.02) (end 145.225 74.02) (width 0.2) (layer B.Cu) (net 10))
 (segment (start 146.74 77.5) (end 146.44 77.8) (width 0.2) (layer F.Cu) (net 10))
 (segment (start 147.3 77.5) (end 146.74 77.5) (width 0.2) (layer F.Cu) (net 10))
 (segment (start 148.29 77.165) (end 147.635 77.165) (width 0.2) (layer F.Cu) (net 10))
 (segment (start 147.635 77.165) (end 147.3 77.5) (width 0.2) (layer F.Cu) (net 10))
 (segment (start 147.159999 74.109999) (end 147.07 74.02) (width 0.2) (layer F.Cu) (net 10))
 (segment (start 147.635 77.165) (end 147.159999 76.689999) (width 0.2) (layer F.Cu) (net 10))
 (segment (start 147.159999 76.689999) (end 147.159999 74.109999) (width 0.2) (layer F.Cu) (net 10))
 (segment (start 134.46 72.88) (end 134.935 72.88) (width 0.2) (layer F.Cu) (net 5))
 (segment (start 137.33 74.91) (end 137.425001 74.814999) (width 0.2) (layer B.Cu) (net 5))
 (segment (start 139.29 73.985) (end 138.255 73.985) (width 0.2) (layer B.Cu) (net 5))
 (segment (start 138.255 73.985) (end 137.974999 74.265001) (width 0.2) (layer B.Cu) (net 5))
 (segment (start 136.555 74.91) (end 137.33 74.91) (width 0.2) (layer B.Cu) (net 5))
 (segment (start 137.425001 74.814999) (end 137.7 74.54) (width 0.2) (layer B.Cu) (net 5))
 (segment (start 137.974999 74.265001) (end 137.7 74.54) (width 0.2) (layer B.Cu) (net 5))
 (via (at 137.7 74.54) (size 0.55) (drill 0.3) (layers F.Cu B.Cu) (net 5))
 (segment (start 138.26 73.98) (end 137.7 74.54) (width 0.2) (layer F.Cu) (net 5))
 (segment (start 138.26 73.27) (end 138.26 73.98) (width 0.2) (layer F.Cu) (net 5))
 (segment (start 137.94 72.95) (end 138.26 73.27) (width 0.2) (layer F.Cu) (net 5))
 (segment (start 135.48 72.95) (end 137.94 72.95) (width 0.2) (layer F.Cu) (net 5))
 (segment (start 134.46 72.88) (end 135.41 72.88) (width 0.2) (layer F.Cu) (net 5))
 (segment (start 135.41 72.88) (end 135.48 72.95) (width 0.2) (layer F.Cu) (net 5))
 (via (at 140.82 71.7) (size 0.55) (drill 0.3) (layers F.Cu B.Cu) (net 4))
 (segment (start 138.34 72.035) (end 139.29 72.035) (width 0.2) (layer B.Cu) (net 4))
 (segment (start 137.365 72.035) (end 138.34 72.035) (width 0.2) (layer B.Cu) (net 4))
 (segment (start 136.96 71.63) (end 137.365 72.035) (width 0.2) (layer B.Cu) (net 4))
 (segment (start 136.565 71.63) (end 136.96 71.63) (width 0.2) (layer B.Cu) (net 4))
 (segment (start 140.485 72.035) (end 140.82 71.7) (width 0.2) (layer B.Cu) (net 4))
 (segment (start 139.29 72.035) (end 140.485 72.035) (width 0.2) (layer B.Cu) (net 4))
 (segment (start 140.154999 73.055001) (end 140.154999 72.365001) (width 0.2) (layer F.Cu) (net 4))
 (segment (start 140.545001 71.974999) (end 140.82 71.7) (width 0.2) (layer F.Cu) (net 4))
 (segment (start 136.8 75.46) (end 137.75 75.46) (width 0.2) (layer F.Cu) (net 4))
 (segment (start 140.154999 72.365001) (end 140.545001 71.974999) (width 0.2) (layer F.Cu) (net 4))
 (segment (start 137.75 75.46) (end 140.154999 73.055001) (width 0.2) (layer F.Cu) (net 4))
 (segment (start 142.73 69.68) (end 142.73 70.54) (width 0.2) (layer F.Cu) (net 14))
 (segment (start 145.19 71.385) (end 143.575 71.385) (width 0.2) (layer B.Cu) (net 14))
 (segment (start 142.73 70.54) (end 143.275001 71.085001) (width 0.2) (layer F.Cu) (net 14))
 (segment (start 143.275001 71.085001) (end 143.55 71.36) (width 0.2) (layer F.Cu) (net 14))
 (segment (start 143.575 71.385) (end 143.55 71.36) (width 0.2) (layer B.Cu) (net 14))
 (via (at 143.55 71.36) (size 0.55) (drill 0.3) (layers F.Cu B.Cu) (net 14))
 (via (at 140.68 74.67) (size 0.55) (drill 0.3) (layers F.Cu B.Cu) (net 2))
 (segment (start 139.325 74.67) (end 139.29 74.635) (width 0.2) (layer B.Cu) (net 2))
 (segment (start 140.68 74.67) (end 139.325 74.67) (width 0.2) (layer B.Cu) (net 2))
 (segment (start 140.91 69.72) (end 140.21 69.72) (width 0.2) (layer F.Cu) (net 2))
 (segment (start 141.395001 70.205001) (end 140.91 69.72) (width 0.2) (layer F.Cu) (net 2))
 (segment (start 141.395001 73.954999) (end 141.395001 70.205001) (width 0.2) (layer F.Cu) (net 2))
 (segment (start 140.68 74.67) (end 141.395001 73.954999) (width 0.2) (layer F.Cu) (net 2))
 (segment (start 140.21 69.72) (end 140.21 69.72) (width 0.2) (layer F.Cu) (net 2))
 (segment (start 135.595 75.95) (end 135.595 76.759302) (width 0.2) (layer B.Cu) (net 2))
 (segment (start 135.595 76.759302) (end 136.344999 77.509301) (width 0.2) (layer B.Cu) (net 2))
 (segment (start 136.359301 77.509301) (end 136.78999 77.93999) (width 0.2) (layer B.Cu) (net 2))
 (segment (start 136.344999 77.509301) (end 136.359301 77.509301) (width 0.2) (layer B.Cu) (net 2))
 (segment (start 140.954999 74.395001) (end 140.68 74.67) (width 0.2) (layer B.Cu) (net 2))
 (segment (start 141.596003 74.395001) (end 140.954999 74.395001) (width 0.2) (layer B.Cu) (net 2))
 (segment (start 142.145001 74.943999) (end 141.596003 74.395001) (width 0.2) (layer B.Cu) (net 2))
 (segment (start 142.145001 75.496001) (end 142.145001 74.943999) (width 0.2) (layer B.Cu) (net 2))
 (segment (start 139.701012 77.93999) (end 142.145001 75.496001) (width 0.2) (layer B.Cu) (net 2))
 (segment (start 136.78999 77.93999) (end 139.701012 77.93999) (width 0.2) (layer B.Cu) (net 2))
 (via (at 147.639998 71.08) (size 0.55) (drill 0.3) (layers F.Cu B.Cu) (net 12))
 (segment (start 145.19 72.035) (end 146.684998 72.035) (width 0.2) (layer B.Cu) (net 12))
 (segment (start 146.684998 72.035) (end 147.364999 71.354999) (width 0.2) (layer B.Cu) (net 12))
 (segment (start 147.364999 71.354999) (end 147.639998 71.08) (width 0.2) (layer B.Cu) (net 12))
 (segment (start 147.8 69.66) (end 147.8 70.919998) (width 0.2) (layer F.Cu) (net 12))
 (segment (start 147.8 70.919998) (end 147.639998 71.08) (width 0.2) (layer F.Cu) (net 12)))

